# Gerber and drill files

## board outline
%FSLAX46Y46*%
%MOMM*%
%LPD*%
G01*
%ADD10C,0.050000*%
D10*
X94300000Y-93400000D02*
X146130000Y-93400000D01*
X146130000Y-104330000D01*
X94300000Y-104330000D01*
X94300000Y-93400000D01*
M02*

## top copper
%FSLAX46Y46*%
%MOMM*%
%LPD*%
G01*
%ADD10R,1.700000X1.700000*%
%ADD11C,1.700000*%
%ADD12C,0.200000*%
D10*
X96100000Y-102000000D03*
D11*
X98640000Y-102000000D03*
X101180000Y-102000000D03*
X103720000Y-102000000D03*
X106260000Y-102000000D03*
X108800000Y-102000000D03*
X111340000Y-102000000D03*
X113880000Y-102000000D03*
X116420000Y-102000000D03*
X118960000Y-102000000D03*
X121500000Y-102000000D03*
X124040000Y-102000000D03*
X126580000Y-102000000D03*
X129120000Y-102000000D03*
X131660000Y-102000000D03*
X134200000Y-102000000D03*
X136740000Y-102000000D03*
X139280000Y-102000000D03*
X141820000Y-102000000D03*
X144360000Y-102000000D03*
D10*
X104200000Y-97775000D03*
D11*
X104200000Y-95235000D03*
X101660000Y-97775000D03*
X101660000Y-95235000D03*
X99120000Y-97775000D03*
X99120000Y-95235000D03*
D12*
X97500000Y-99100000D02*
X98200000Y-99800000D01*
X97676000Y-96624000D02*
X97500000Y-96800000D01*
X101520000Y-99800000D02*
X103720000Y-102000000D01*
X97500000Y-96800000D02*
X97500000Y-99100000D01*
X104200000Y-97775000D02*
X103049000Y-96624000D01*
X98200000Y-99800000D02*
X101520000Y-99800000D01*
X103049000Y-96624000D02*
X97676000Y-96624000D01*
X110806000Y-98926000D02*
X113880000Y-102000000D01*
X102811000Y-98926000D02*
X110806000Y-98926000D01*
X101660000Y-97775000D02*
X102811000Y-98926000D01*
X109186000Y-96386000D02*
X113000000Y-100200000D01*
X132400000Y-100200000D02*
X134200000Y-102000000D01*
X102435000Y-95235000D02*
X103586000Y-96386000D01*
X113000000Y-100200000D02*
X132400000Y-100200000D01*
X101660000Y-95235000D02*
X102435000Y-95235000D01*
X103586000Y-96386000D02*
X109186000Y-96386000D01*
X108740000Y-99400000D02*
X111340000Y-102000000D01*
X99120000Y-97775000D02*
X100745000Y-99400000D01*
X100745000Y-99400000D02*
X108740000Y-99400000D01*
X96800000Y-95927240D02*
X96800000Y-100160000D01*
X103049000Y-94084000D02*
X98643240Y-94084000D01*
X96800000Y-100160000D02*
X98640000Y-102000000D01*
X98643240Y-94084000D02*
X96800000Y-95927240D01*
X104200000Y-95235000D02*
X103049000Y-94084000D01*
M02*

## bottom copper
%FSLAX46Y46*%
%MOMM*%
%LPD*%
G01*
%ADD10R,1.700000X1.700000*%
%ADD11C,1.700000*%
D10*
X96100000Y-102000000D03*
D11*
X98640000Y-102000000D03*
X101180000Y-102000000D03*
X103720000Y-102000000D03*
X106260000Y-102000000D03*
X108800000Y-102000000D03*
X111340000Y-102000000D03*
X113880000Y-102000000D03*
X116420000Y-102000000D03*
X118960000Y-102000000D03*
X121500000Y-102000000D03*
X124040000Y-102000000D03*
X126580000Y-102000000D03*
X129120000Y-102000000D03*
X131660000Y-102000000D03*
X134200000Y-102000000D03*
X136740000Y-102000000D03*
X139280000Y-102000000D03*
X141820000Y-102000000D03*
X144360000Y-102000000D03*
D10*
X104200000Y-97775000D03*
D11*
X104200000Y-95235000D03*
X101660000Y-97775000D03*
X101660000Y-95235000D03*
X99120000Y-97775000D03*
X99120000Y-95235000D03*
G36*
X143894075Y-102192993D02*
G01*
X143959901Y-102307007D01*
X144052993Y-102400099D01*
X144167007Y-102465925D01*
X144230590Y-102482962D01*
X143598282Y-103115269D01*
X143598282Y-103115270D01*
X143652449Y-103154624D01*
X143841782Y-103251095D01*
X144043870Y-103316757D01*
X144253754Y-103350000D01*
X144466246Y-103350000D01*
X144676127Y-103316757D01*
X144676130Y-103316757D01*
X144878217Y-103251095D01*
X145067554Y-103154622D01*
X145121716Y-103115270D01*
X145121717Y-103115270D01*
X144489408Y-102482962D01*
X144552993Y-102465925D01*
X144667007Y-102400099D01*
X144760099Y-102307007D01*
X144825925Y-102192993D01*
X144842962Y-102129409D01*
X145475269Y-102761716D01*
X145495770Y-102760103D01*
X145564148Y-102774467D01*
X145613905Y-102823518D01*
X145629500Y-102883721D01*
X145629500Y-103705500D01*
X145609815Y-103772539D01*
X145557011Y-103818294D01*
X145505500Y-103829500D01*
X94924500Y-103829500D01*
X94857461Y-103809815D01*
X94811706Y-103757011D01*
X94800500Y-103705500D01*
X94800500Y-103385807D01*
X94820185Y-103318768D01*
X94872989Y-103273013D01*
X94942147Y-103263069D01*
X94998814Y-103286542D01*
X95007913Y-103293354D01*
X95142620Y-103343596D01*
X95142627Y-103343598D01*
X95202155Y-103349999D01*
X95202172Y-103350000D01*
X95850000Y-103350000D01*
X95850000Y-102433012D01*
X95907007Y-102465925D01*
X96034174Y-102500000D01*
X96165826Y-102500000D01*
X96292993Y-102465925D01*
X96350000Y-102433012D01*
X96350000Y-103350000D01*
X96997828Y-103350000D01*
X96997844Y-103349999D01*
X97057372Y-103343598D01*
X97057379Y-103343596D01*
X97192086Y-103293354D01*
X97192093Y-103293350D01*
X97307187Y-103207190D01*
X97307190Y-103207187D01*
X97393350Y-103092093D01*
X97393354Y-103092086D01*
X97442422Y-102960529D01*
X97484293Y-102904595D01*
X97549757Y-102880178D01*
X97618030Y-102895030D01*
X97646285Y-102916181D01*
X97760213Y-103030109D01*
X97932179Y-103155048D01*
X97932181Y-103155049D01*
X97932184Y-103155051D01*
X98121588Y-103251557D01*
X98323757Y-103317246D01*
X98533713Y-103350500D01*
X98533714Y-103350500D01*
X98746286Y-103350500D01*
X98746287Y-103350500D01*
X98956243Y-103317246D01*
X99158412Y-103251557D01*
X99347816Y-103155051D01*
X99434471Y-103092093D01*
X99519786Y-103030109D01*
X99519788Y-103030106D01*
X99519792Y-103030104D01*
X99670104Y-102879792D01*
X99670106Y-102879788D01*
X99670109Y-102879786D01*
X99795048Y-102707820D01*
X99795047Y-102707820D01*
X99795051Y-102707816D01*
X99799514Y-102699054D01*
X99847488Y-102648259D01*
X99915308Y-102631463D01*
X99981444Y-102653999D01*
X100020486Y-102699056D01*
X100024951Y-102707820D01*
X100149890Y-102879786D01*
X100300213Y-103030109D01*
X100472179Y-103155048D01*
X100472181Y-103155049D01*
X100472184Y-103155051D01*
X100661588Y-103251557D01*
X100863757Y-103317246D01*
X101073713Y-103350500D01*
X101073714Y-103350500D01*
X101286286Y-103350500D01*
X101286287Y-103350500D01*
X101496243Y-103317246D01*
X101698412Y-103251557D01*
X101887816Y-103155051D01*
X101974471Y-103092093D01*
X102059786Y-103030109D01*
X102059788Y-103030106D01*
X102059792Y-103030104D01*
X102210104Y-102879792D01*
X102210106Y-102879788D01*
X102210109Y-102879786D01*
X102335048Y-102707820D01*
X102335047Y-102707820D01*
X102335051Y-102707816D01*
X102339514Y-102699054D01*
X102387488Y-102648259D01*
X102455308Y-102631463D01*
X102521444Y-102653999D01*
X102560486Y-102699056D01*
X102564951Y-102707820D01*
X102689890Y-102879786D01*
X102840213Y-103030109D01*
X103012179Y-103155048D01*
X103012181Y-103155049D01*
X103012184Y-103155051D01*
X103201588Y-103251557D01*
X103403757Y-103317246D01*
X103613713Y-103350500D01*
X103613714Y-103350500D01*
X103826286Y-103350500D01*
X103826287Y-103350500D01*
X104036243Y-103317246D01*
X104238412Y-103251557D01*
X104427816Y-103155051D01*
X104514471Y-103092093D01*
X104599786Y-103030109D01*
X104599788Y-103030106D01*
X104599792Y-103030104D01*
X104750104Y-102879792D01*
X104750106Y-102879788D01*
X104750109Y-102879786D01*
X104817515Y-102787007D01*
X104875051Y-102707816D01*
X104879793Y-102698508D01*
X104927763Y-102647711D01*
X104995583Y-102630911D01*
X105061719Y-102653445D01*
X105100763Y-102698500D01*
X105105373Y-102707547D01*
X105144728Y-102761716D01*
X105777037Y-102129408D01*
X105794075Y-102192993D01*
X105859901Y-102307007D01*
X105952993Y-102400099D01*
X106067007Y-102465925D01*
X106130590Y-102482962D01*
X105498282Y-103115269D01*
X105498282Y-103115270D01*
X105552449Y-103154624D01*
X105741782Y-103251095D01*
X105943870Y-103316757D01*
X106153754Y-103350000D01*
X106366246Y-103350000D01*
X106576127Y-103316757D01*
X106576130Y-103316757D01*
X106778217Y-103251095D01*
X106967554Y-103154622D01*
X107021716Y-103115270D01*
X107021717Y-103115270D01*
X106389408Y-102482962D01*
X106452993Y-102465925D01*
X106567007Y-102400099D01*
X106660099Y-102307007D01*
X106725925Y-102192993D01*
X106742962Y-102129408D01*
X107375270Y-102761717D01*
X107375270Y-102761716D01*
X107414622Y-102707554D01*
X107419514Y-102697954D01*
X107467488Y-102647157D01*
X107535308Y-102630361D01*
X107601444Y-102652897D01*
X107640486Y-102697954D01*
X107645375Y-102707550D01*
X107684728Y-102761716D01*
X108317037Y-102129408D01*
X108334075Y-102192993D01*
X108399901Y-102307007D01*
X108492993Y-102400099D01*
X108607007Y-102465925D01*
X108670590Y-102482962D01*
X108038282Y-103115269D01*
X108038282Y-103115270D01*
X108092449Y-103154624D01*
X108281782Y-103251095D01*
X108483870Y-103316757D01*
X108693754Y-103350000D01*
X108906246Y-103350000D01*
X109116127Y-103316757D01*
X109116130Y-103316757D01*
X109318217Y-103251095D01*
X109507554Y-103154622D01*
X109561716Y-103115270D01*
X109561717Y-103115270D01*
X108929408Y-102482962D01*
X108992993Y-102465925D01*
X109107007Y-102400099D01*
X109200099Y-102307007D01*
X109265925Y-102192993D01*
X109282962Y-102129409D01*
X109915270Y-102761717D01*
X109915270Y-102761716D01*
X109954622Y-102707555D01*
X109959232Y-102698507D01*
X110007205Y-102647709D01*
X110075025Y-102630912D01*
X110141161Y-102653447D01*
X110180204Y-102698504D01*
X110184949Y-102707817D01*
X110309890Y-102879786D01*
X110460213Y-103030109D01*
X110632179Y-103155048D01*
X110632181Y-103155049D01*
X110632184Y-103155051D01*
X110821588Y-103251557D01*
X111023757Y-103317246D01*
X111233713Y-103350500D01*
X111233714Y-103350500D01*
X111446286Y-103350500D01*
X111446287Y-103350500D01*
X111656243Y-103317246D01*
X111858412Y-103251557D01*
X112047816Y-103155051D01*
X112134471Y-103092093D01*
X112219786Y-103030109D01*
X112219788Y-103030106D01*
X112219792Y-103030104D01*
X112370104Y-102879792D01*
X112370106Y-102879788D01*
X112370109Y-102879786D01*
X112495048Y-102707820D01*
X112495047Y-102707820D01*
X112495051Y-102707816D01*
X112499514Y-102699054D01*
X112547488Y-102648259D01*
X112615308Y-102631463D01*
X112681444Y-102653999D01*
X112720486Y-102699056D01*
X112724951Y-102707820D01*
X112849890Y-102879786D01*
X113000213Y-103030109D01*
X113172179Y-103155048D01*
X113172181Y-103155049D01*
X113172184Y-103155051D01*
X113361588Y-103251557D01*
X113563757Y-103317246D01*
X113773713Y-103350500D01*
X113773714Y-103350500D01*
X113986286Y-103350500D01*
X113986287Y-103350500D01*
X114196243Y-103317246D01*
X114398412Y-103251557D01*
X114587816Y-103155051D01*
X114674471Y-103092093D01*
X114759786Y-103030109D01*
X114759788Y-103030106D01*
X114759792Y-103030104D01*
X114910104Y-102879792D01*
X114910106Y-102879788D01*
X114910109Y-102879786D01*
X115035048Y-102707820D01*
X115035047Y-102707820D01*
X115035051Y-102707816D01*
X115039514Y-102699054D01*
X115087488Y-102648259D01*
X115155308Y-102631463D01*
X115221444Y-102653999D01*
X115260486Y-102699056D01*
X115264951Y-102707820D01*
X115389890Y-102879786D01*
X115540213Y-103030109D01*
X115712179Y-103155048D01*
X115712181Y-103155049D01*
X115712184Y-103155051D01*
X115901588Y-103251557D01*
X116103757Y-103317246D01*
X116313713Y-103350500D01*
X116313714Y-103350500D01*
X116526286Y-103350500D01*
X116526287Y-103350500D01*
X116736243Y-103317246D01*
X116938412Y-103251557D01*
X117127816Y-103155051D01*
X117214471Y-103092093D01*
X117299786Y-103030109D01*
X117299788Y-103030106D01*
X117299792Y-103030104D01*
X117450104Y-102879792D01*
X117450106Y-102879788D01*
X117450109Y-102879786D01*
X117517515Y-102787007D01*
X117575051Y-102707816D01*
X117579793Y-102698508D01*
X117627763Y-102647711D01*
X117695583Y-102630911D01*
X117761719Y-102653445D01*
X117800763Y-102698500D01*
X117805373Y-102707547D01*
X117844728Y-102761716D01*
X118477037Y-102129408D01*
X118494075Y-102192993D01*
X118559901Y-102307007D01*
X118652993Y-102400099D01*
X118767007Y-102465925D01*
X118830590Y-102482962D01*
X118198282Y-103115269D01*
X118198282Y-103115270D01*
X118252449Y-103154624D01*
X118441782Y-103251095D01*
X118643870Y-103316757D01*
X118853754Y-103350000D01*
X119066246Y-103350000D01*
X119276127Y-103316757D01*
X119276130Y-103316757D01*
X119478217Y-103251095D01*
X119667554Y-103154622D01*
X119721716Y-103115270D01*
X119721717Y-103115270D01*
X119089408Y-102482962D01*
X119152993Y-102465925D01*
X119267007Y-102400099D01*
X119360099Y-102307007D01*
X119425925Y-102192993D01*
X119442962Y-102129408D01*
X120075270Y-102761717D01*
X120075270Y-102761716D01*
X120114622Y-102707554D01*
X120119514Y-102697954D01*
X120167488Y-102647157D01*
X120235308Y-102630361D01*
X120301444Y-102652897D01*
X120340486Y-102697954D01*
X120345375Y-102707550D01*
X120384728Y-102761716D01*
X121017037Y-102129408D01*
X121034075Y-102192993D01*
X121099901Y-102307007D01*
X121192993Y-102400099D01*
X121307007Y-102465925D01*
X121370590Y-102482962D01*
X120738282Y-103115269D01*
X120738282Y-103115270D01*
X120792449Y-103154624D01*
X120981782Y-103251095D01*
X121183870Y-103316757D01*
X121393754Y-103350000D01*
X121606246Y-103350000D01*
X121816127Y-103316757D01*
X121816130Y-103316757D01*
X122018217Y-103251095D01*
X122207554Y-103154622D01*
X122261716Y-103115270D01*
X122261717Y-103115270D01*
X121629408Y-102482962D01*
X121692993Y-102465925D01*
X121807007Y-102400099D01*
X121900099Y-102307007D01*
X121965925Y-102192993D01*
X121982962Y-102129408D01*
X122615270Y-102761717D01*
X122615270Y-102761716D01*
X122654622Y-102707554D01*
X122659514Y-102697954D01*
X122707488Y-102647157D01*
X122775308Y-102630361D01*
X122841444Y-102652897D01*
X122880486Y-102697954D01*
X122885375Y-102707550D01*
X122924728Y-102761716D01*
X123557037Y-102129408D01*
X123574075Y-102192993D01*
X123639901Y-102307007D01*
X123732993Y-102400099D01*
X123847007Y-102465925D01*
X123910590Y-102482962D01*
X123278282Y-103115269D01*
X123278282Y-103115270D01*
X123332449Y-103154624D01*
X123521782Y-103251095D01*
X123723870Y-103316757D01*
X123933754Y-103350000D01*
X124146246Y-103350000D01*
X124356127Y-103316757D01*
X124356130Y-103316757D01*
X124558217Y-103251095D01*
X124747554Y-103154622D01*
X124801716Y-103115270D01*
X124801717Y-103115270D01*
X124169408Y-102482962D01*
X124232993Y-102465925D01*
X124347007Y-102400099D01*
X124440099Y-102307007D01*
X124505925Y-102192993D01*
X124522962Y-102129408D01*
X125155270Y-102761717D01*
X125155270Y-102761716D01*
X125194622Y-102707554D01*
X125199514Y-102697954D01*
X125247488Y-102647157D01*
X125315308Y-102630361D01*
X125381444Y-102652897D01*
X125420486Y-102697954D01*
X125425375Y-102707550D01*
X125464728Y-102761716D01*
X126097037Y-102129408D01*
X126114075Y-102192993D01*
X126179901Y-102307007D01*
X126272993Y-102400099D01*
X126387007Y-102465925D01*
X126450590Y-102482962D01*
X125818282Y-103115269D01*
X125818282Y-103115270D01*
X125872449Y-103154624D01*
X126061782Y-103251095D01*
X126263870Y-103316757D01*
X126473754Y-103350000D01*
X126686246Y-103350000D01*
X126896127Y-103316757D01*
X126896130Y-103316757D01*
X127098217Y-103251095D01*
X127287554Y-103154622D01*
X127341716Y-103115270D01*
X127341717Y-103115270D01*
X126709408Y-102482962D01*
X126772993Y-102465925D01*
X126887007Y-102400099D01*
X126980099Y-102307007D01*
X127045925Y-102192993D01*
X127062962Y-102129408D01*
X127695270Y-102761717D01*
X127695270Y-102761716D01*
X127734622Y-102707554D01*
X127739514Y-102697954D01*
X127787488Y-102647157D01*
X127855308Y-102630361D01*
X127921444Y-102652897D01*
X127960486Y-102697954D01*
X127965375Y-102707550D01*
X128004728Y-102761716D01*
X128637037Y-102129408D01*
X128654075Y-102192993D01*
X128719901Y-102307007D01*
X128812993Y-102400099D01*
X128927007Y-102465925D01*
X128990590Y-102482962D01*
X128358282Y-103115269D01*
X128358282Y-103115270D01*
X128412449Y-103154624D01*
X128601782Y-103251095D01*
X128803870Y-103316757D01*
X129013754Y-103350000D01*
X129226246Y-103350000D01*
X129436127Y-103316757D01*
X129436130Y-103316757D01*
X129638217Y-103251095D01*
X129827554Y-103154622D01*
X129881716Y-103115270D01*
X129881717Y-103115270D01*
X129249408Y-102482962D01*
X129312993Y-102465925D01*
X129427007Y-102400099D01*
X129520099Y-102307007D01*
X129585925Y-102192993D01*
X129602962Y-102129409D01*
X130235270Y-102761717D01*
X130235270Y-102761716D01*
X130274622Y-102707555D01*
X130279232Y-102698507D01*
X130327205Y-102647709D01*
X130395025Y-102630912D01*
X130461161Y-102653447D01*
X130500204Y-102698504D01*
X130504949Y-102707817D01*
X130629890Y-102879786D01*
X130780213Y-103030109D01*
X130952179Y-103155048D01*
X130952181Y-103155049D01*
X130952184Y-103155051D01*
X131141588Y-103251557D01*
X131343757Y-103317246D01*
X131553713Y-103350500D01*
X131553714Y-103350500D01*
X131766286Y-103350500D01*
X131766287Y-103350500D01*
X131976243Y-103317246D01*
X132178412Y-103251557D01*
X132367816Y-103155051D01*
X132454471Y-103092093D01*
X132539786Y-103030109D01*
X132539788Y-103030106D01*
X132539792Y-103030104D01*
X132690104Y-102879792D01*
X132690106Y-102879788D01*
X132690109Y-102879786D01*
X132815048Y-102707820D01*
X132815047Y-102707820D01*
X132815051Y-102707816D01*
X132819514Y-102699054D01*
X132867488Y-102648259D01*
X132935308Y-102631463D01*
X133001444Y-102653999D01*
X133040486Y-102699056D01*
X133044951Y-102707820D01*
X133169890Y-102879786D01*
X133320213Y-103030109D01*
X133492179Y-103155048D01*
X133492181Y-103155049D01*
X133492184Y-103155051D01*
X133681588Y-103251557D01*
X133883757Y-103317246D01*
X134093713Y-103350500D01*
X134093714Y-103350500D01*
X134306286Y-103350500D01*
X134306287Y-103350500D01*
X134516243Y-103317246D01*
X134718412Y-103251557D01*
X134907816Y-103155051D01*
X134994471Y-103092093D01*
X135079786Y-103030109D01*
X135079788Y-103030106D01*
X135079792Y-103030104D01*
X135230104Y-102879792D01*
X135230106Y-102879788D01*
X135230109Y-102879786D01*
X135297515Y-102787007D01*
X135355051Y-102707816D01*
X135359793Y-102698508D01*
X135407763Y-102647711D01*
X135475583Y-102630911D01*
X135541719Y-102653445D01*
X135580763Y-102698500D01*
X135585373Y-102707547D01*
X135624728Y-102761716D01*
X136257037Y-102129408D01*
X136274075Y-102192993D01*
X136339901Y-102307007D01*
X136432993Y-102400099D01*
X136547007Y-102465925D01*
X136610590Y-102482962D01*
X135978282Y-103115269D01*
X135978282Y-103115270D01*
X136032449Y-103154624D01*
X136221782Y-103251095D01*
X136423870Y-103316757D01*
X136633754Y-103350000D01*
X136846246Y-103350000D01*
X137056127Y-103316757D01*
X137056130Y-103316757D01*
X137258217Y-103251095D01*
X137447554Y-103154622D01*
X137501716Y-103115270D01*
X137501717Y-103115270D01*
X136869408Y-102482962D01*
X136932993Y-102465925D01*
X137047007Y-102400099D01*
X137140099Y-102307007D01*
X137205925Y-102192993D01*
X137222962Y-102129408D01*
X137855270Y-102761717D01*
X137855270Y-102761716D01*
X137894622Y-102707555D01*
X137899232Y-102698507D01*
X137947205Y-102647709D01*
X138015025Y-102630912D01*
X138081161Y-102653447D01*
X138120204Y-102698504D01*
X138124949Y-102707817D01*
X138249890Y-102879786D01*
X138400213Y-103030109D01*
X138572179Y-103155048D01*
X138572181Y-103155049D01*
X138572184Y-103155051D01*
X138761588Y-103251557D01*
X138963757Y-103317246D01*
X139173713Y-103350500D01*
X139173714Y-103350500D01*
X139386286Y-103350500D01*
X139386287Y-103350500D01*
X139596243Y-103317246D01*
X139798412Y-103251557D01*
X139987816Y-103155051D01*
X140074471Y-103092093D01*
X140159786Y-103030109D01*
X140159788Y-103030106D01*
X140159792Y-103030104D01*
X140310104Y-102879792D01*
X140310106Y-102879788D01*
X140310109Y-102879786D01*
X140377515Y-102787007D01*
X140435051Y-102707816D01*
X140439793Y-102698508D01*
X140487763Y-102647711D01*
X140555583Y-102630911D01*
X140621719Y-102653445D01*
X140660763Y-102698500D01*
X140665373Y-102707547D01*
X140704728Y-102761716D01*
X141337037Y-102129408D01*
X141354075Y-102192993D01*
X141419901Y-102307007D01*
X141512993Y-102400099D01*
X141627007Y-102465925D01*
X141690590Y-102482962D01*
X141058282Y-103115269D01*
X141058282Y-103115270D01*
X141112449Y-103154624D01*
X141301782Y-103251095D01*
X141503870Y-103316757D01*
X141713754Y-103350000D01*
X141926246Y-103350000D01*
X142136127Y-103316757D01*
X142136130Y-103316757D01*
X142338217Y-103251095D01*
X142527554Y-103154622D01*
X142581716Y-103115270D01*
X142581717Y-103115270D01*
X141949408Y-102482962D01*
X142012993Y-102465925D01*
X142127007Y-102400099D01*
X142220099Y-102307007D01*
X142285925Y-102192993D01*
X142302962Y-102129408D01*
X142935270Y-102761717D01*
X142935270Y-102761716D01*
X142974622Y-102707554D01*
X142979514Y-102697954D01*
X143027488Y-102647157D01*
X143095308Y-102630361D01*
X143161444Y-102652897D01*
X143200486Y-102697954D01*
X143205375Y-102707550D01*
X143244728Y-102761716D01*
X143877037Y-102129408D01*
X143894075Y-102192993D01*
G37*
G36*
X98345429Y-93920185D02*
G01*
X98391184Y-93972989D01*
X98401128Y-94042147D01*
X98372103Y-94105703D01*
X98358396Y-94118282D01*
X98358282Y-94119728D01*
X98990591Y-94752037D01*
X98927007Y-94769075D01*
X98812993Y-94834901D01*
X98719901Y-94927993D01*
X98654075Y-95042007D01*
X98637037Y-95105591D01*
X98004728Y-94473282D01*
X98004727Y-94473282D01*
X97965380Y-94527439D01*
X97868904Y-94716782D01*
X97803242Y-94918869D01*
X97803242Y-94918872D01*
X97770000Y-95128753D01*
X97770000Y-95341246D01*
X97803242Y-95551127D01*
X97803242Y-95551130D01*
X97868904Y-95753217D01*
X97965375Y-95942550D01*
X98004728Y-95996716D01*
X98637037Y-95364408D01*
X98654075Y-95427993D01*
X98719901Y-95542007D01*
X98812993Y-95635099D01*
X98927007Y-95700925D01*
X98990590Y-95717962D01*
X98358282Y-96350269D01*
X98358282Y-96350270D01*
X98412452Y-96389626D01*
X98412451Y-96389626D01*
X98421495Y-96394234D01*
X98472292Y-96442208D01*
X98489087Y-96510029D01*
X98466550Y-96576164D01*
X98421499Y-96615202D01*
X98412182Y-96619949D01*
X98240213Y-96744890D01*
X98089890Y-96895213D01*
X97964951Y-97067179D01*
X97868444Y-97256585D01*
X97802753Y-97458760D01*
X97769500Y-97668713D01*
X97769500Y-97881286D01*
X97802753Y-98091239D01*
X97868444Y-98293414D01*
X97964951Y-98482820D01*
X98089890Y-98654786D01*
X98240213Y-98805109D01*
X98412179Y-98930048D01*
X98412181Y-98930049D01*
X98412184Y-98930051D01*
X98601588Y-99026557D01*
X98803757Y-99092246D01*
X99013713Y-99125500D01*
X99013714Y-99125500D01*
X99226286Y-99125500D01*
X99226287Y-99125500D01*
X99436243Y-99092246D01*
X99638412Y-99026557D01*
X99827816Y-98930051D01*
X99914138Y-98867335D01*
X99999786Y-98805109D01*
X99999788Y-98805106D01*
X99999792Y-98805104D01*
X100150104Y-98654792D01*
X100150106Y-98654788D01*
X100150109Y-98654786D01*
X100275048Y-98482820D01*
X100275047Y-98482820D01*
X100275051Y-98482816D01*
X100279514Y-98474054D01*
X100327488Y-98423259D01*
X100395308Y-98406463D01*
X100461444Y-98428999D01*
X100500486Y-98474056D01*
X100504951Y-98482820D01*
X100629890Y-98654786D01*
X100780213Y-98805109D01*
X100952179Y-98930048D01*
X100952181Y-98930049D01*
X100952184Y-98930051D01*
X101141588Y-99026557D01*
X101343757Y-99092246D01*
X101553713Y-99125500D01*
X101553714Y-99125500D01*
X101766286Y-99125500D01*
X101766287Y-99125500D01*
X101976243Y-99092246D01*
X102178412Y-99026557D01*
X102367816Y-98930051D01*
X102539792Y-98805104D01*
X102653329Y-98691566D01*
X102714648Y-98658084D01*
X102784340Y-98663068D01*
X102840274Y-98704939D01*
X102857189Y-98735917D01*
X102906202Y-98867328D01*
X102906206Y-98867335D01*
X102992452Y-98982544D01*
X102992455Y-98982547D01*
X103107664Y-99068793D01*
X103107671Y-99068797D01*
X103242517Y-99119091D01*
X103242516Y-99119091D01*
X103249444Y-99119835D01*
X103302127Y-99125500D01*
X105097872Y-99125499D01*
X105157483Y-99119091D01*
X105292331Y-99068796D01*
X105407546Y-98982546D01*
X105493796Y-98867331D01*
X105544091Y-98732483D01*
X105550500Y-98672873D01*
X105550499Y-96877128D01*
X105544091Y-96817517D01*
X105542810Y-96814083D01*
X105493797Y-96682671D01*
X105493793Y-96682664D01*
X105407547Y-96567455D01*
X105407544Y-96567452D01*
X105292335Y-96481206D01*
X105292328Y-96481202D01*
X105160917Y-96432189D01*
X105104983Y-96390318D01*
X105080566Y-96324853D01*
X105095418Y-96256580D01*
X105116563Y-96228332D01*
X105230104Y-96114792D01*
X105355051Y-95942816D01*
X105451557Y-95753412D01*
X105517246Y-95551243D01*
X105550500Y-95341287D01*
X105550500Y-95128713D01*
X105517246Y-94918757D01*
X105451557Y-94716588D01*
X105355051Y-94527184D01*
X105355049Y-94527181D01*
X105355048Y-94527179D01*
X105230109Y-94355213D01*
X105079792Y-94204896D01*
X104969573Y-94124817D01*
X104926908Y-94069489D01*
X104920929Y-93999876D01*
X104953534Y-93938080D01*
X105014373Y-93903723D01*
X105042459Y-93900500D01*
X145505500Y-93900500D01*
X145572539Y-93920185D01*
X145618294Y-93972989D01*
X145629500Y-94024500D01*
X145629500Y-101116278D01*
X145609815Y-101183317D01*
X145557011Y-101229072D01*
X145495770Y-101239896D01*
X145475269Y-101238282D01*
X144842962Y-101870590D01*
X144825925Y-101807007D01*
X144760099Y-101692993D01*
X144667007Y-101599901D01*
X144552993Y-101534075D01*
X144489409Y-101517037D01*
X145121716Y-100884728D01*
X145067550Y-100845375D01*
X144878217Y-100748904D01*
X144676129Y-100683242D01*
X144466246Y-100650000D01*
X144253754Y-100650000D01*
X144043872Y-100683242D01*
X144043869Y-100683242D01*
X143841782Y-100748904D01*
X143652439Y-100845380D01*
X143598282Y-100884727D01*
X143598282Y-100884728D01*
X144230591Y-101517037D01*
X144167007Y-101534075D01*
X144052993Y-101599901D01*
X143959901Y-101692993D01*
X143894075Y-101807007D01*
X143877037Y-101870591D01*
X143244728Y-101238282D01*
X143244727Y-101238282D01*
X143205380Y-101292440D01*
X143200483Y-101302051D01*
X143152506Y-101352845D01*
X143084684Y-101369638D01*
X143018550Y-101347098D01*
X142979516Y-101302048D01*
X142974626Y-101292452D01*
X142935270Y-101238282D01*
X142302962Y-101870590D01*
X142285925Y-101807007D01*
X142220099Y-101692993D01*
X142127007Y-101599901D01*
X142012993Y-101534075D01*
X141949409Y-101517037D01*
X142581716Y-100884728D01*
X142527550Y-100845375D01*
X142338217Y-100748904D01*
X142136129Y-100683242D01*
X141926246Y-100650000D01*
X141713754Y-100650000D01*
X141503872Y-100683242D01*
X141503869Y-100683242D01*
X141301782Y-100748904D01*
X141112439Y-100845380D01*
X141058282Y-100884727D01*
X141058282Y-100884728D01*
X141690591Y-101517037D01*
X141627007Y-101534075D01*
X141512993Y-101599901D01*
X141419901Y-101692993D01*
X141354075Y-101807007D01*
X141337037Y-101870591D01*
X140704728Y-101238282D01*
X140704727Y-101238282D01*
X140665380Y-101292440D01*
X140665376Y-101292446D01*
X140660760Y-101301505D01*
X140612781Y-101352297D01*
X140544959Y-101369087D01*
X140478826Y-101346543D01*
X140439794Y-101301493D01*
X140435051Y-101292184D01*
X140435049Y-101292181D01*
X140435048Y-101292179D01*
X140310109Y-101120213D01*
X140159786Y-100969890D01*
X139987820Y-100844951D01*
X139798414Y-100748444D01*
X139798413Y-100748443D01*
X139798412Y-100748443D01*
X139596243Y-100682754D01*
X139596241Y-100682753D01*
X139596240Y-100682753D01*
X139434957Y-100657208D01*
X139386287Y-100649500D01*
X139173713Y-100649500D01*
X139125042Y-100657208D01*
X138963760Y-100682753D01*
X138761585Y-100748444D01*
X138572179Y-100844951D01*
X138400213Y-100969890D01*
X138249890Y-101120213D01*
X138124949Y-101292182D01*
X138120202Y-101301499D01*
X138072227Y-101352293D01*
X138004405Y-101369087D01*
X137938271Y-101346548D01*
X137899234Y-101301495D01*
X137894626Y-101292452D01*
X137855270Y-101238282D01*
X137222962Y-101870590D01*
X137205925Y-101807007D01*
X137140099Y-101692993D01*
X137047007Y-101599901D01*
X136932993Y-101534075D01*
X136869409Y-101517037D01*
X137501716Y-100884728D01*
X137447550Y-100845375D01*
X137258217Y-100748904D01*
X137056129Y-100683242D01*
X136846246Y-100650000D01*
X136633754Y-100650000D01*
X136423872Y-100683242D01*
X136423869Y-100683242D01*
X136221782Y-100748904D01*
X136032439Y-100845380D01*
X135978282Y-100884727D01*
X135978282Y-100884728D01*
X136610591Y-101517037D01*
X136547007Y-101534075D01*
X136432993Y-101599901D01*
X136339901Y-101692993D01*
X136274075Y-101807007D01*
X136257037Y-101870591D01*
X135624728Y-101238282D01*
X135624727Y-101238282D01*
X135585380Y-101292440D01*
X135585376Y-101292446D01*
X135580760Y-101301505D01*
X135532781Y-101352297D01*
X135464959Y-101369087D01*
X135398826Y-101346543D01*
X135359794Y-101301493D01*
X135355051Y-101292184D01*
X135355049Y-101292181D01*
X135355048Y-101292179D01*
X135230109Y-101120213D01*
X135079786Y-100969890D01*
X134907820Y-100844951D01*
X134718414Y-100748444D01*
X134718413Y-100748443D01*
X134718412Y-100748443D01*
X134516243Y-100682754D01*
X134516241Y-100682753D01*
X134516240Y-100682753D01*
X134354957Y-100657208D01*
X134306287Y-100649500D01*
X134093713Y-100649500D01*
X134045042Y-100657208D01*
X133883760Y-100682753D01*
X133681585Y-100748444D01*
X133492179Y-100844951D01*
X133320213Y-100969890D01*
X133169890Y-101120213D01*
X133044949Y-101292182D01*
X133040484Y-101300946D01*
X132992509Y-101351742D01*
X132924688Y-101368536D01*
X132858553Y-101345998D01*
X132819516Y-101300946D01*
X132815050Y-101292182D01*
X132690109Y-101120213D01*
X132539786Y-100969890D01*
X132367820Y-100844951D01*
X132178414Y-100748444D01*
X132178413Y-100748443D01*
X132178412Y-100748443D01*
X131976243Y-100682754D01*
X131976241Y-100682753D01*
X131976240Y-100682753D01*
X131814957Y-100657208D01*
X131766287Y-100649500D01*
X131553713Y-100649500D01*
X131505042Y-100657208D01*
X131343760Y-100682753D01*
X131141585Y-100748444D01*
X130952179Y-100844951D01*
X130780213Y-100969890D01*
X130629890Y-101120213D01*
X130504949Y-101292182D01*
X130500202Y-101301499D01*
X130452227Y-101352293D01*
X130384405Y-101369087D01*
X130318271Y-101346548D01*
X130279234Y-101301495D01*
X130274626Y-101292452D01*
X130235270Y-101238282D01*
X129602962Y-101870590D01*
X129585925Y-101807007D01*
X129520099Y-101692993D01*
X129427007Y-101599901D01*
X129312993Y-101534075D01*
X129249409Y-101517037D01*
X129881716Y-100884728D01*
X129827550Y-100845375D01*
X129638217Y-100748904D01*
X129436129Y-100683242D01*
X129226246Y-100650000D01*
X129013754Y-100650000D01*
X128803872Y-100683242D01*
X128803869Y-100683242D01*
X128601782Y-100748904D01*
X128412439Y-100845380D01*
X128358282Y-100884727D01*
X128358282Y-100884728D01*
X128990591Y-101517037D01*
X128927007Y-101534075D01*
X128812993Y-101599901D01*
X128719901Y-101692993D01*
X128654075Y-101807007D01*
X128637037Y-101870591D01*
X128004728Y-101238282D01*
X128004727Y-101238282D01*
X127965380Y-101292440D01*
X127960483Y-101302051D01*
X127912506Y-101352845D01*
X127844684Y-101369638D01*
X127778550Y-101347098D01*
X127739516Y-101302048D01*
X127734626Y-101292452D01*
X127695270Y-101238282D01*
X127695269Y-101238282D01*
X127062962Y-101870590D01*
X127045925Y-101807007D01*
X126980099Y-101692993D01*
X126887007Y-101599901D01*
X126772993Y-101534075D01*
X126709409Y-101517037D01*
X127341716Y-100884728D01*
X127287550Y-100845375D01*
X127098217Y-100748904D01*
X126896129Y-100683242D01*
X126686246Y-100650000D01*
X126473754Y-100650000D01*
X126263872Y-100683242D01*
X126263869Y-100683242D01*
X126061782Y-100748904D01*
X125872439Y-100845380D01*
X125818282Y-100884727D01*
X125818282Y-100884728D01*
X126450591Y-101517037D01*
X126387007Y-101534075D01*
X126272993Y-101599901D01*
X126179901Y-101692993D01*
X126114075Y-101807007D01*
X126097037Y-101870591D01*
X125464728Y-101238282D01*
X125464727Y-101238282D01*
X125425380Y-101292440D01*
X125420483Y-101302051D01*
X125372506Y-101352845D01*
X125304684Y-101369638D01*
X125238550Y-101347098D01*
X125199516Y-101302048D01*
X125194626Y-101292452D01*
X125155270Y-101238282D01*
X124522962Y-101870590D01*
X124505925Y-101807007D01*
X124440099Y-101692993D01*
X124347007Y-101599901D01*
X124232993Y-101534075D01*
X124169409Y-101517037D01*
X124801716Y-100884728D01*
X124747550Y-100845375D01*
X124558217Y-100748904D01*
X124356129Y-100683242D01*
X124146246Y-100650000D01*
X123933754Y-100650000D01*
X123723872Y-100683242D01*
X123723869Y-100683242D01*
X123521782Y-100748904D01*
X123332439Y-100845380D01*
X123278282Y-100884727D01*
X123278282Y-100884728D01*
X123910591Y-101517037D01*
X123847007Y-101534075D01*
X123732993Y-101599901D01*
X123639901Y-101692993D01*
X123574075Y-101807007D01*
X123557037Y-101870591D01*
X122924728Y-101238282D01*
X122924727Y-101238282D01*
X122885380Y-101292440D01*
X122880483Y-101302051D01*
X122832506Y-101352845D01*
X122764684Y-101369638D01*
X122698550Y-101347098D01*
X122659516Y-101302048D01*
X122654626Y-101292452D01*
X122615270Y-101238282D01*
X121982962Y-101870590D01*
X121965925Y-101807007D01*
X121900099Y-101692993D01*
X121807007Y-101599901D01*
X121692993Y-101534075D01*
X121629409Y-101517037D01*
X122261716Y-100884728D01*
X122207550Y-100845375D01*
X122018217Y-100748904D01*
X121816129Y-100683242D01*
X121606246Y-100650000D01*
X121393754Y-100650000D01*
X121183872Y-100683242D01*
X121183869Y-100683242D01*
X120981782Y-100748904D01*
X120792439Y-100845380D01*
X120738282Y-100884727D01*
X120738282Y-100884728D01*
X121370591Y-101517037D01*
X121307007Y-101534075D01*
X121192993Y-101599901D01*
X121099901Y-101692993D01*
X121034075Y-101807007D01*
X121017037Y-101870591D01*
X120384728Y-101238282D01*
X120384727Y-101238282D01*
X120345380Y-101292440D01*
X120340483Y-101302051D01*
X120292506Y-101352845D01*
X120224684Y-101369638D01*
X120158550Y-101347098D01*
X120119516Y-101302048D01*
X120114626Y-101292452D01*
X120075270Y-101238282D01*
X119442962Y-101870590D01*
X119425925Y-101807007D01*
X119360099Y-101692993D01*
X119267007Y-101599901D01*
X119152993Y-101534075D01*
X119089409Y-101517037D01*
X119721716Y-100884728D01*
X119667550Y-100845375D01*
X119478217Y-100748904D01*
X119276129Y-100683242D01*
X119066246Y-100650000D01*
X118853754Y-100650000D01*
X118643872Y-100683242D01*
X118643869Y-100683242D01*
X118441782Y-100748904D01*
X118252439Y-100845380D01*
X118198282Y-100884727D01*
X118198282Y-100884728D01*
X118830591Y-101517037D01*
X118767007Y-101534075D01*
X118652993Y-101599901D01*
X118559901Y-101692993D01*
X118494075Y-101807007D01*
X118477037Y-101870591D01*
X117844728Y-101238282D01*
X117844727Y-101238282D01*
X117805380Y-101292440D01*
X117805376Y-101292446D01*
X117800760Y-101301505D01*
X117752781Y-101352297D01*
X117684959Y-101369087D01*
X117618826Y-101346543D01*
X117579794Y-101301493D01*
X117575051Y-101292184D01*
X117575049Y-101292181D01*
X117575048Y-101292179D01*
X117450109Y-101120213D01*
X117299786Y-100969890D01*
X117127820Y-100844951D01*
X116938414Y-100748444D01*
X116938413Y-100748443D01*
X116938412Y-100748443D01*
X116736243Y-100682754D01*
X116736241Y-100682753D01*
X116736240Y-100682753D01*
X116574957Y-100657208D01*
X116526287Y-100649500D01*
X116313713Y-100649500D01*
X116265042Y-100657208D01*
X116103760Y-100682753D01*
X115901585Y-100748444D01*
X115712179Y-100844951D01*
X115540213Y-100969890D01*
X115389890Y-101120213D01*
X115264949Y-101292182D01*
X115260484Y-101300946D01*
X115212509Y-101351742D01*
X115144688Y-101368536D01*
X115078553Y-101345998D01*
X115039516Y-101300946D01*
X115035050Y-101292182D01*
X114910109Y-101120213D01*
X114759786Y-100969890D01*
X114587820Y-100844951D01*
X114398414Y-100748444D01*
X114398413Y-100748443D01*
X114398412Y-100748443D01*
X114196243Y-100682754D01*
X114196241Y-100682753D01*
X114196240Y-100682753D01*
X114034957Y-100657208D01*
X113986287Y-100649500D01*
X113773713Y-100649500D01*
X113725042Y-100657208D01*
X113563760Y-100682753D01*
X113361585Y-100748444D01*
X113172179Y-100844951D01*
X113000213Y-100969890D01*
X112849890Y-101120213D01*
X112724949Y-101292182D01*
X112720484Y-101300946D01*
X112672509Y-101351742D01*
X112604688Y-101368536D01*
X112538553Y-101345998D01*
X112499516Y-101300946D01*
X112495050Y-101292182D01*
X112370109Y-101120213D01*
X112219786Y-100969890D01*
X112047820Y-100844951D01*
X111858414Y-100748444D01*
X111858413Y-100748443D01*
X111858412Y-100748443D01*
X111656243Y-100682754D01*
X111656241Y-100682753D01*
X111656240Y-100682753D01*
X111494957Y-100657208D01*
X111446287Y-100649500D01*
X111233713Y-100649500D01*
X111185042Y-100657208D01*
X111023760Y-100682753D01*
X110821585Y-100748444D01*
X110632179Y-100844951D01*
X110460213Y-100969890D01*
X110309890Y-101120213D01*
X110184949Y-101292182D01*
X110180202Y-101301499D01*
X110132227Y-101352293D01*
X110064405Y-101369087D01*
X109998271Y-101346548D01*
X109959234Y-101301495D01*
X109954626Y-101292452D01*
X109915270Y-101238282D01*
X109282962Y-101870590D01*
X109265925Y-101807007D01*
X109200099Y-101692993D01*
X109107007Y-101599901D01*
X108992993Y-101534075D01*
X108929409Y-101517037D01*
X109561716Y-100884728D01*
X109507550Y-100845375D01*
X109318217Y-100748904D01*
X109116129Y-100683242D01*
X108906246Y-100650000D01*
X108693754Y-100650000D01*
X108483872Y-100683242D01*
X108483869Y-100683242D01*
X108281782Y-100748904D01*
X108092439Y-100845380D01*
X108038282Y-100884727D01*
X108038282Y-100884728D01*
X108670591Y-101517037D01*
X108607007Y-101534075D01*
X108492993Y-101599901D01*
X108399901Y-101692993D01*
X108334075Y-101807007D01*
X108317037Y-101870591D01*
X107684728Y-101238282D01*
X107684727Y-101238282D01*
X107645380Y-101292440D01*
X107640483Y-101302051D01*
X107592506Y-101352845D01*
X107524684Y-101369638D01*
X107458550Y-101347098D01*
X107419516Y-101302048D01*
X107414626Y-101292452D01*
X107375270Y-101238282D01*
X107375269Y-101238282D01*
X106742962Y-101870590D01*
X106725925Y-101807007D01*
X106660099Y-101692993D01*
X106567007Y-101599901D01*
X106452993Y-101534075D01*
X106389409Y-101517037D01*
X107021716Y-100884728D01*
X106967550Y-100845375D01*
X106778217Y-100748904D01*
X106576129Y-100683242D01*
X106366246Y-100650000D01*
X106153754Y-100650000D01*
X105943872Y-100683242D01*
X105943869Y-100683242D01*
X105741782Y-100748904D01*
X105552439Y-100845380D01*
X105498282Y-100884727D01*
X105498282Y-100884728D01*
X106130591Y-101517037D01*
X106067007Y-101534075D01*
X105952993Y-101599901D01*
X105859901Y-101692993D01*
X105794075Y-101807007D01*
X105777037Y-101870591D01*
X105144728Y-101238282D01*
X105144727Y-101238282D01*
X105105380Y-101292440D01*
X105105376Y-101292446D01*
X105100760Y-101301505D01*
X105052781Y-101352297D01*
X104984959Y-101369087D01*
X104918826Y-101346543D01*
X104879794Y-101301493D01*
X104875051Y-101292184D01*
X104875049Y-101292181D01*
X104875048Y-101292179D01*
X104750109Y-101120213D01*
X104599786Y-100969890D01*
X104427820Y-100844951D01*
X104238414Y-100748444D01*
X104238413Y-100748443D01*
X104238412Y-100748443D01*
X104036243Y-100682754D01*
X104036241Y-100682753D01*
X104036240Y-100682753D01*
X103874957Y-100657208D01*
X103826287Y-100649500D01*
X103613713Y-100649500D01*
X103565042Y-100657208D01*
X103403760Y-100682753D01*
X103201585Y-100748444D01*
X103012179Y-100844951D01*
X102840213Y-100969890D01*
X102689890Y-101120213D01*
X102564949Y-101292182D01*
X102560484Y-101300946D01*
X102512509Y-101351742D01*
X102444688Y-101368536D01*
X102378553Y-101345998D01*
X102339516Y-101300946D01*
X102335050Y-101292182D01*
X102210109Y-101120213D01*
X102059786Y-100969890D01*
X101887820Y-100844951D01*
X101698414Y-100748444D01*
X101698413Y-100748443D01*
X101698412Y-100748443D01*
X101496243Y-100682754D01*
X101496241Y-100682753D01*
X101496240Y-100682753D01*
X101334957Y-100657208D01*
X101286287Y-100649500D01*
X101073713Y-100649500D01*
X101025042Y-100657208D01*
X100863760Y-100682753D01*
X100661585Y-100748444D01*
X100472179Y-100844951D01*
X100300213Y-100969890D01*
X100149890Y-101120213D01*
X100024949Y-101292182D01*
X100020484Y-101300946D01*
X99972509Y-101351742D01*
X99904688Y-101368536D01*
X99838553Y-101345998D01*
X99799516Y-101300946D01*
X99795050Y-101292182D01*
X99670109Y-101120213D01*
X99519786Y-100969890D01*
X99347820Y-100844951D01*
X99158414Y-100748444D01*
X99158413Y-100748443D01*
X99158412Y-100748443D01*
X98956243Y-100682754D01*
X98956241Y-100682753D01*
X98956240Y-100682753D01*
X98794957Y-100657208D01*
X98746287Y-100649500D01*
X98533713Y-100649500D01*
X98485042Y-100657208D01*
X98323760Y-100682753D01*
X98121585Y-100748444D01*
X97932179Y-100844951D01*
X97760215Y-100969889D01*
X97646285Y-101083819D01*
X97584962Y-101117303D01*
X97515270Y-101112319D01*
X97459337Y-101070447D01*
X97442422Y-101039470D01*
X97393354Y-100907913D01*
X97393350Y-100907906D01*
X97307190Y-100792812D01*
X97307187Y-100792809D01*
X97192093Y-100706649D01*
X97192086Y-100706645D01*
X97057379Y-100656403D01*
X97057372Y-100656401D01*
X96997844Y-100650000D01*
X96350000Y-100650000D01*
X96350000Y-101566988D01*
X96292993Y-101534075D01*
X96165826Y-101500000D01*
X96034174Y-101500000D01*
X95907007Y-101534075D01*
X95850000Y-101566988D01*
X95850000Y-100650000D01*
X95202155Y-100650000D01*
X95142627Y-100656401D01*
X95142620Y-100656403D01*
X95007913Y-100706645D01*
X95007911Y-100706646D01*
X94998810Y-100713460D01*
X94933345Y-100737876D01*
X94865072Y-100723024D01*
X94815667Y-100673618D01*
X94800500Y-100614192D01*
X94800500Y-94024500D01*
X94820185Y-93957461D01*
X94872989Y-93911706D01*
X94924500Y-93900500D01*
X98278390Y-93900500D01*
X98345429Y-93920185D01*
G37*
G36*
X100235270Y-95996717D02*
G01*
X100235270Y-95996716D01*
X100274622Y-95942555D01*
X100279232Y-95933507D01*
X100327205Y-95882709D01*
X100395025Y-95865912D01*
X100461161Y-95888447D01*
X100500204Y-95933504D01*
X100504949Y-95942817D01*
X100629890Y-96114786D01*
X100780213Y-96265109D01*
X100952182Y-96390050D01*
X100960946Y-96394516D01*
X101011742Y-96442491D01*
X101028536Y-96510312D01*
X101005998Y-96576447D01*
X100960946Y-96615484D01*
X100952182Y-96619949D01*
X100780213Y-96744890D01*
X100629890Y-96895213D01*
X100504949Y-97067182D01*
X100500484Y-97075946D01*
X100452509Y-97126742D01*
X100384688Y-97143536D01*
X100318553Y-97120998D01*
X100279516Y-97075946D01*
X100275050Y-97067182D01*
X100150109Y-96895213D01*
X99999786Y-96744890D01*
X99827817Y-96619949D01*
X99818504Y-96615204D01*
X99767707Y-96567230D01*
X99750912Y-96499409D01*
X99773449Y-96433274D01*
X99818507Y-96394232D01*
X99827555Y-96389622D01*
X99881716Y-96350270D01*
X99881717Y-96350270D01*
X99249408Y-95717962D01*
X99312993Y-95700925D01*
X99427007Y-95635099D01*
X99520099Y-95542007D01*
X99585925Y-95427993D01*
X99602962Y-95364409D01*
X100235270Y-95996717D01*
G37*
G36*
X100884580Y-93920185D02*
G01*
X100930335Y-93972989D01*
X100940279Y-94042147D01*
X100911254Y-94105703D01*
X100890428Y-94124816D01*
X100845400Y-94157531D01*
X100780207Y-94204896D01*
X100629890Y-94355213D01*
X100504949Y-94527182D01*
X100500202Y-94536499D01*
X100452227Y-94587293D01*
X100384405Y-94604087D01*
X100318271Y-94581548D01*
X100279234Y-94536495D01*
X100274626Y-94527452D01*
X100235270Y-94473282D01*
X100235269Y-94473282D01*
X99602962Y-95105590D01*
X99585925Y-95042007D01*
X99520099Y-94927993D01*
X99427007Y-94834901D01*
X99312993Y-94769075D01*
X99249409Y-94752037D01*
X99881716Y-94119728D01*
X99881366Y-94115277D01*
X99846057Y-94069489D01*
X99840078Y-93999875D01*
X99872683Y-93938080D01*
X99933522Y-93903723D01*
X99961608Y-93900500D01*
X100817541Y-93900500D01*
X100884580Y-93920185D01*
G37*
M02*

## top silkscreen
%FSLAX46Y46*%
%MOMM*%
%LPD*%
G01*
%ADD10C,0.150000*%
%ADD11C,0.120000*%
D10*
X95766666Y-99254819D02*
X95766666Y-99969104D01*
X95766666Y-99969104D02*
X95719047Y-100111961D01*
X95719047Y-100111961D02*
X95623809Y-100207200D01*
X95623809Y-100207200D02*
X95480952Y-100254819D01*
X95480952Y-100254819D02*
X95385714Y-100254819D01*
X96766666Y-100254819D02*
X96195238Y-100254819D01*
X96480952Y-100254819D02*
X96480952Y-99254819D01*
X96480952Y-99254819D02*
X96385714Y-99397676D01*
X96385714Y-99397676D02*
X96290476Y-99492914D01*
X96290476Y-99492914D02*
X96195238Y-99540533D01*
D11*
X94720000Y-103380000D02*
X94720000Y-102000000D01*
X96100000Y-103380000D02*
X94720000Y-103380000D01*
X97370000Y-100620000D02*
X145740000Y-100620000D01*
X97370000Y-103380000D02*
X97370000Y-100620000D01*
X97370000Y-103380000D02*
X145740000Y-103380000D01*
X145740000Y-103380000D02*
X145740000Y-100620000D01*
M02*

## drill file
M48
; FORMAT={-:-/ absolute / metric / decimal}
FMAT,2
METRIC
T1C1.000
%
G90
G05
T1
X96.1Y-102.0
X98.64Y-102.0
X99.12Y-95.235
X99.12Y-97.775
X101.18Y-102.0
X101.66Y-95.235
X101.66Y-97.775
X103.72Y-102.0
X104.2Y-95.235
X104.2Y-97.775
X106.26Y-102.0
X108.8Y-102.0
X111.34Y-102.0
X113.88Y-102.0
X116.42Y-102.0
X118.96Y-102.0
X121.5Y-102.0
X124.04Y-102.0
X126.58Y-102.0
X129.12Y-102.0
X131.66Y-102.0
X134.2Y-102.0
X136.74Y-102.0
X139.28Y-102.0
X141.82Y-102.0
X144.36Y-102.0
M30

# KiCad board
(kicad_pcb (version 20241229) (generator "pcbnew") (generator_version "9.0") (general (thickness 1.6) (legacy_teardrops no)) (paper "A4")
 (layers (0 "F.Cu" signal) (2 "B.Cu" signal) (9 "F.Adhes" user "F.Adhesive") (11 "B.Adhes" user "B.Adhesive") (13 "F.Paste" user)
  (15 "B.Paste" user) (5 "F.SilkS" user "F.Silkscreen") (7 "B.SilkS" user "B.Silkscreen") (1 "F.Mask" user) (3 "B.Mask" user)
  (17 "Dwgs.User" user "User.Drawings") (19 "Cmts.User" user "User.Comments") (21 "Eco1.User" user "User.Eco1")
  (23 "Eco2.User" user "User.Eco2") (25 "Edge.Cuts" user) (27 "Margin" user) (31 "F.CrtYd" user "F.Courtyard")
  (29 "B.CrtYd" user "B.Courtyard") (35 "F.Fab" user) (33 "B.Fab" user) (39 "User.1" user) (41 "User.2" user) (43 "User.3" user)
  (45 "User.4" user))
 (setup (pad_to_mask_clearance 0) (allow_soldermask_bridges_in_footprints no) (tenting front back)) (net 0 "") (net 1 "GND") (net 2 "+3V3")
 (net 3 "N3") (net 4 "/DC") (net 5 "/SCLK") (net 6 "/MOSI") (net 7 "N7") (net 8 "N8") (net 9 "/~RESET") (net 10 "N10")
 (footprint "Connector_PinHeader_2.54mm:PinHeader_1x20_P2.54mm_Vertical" (layer "F.Cu") (at 96.1 102 90)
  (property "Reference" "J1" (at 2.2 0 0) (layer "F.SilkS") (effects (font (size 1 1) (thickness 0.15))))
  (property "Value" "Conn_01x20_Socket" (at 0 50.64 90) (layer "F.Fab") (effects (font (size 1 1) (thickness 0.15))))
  (fp_line (start -1.38 -1.38) (end 0 -1.38) (stroke (width 0.12) (type solid)) (layer "F.SilkS"))
  (fp_line (start -1.38 0) (end -1.38 -1.38) (stroke (width 0.12) (type solid)) (layer "F.SilkS"))
  (fp_line (start 1.38 1.27) (end 1.38 49.64) (stroke (width 0.12) (type solid)) (layer "F.SilkS"))
  (fp_line (start -1.38 1.27) (end 1.38 1.27) (stroke (width 0.12) (type solid)) (layer "F.SilkS"))
  (fp_line (start -1.38 1.27) (end -1.38 49.64) (stroke (width 0.12) (type solid)) (layer "F.SilkS"))
  (fp_line (start -1.38 49.64) (end 1.38 49.64) (stroke (width 0.12) (type solid)) (layer "F.SilkS"))
  (pad "1" thru_hole rect (at 0 0 90) (size 1.7 1.7) (drill 1) (layers "*.Cu" "*.Mask") (remove_unused_layers no) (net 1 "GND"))
  (pad "2" thru_hole circle (at 0 2.54 90) (size 1.7 1.7) (drill 1) (layers "*.Cu" "*.Mask") (remove_unused_layers no) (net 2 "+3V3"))
  (pad "3" thru_hole circle (at 0 5.08 90) (size 1.7 1.7) (drill 1) (layers "*.Cu" "*.Mask") (remove_unused_layers no) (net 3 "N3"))
  (pad "4" thru_hole circle (at 0 7.62 90) (size 1.7 1.7) (drill 1) (layers "*.Cu" "*.Mask") (remove_unused_layers no) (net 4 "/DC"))
  (pad "5" thru_hole circle (at 0 10.16 90) (size 1.7 1.7) (drill 1) (layers "*.Cu" "*.Mask") (remove_unused_layers no) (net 1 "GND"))
  (pad "6" thru_hole circle (at 0 12.7 90) (size 1.7 1.7) (drill 1) (layers "*.Cu" "*.Mask") (remove_unused_layers no) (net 1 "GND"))
  (pad "7" thru_hole circle (at 0 15.24 90) (size 1.7 1.7) (drill 1) (layers "*.Cu" "*.Mask") (remove_unused_layers no) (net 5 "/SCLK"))
  (pad "8" thru_hole circle (at 0 17.78 90) (size 1.7 1.7) (drill 1) (layers "*.Cu" "*.Mask") (remove_unused_layers no) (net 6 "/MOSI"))
  (pad "9" thru_hole circle (at 0 20.32 90) (size 1.7 1.7) (drill 1) (layers "*.Cu" "*.Mask") (remove_unused_layers no) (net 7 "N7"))
  (pad "10" thru_hole circle (at 0 22.86 90) (size 1.7 1.7) (drill 1) (layers "*.Cu" "*.Mask") (remove_unused_layers no) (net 1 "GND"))
  (pad "11" thru_hole circle (at 0 25.4 90) (size 1.7 1.7) (drill 1) (layers "*.Cu" "*.Mask") (remove_unused_layers no) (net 1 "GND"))
  (pad "12" thru_hole circle (at 0 27.94 90) (size 1.7 1.7) (drill 1) (layers "*.Cu" "*.Mask") (remove_unused_layers no) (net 1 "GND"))
  (pad "13" thru_hole circle (at 0 30.48 90) (size 1.7 1.7) (drill 1) (layers "*.Cu" "*.Mask") (remove_unused_layers no) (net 1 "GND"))
  (pad "14" thru_hole circle (at 0 33.02 90) (size 1.7 1.7) (drill 1) (layers "*.Cu" "*.Mask") (remove_unused_layers no) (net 1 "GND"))
  (pad "15" thru_hole circle (at 0 35.56 90) (size 1.7 1.7) (drill 1) (layers "*.Cu" "*.Mask") (remove_unused_layers no) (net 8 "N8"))
  (pad "16" thru_hole circle (at 0 38.1 90) (size 1.7 1.7) (drill 1) (layers "*.Cu" "*.Mask") (remove_unused_layers no) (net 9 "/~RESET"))
  (pad "17" thru_hole circle (at 0 40.64 90) (size 1.7 1.7) (drill 1) (layers "*.Cu" "*.Mask") (remove_unused_layers no) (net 1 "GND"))
  (pad "18" thru_hole circle (at 0 43.18 90) (size 1.7 1.7) (drill 1) (layers "*.Cu" "*.Mask") (remove_unused_layers no) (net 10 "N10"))
  (pad "19" thru_hole circle (at 0 45.72 90) (size 1.7 1.7) (drill 1) (layers "*.Cu" "*.Mask") (remove_unused_layers no) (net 1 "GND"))
  (pad "20" thru_hole circle (at 0 48.26 90) (size 1.7 1.7) (drill 1) (layers "*.Cu" "*.Mask") (remove_unused_layers no) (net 1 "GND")))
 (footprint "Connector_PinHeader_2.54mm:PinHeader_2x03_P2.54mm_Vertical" (layer "B.Cu") (at 104.2 97.775 90)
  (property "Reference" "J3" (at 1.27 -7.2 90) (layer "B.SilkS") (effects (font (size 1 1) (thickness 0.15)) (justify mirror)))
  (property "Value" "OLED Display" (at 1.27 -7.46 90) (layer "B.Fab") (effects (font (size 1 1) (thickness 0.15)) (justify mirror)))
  (pad "1" thru_hole rect (at 0 0 90) (size 1.7 1.7) (drill 1) (layers "*.Cu" "*.Mask") (remove_unused_layers no) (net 4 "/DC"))
  (pad "2" thru_hole circle (at 2.54 0 90) (size 1.7 1.7) (drill 1) (layers "*.Cu" "*.Mask") (remove_unused_layers no) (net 2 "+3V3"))
  (pad "3" thru_hole circle (at 0 -2.54 90) (size 1.7 1.7) (drill 1) (layers "*.Cu" "*.Mask") (remove_unused_layers no) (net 6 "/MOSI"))
  (pad "4" thru_hole circle (at 2.54 -2.54 90) (size 1.7 1.7) (drill 1) (layers "*.Cu" "*.Mask") (remove_unused_layers no) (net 9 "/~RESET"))
  (pad "5" thru_hole circle (at 0 -5.08 90) (size 1.7 1.7) (drill 1) (layers "*.Cu" "*.Mask") (remove_unused_layers no) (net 5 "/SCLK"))
  (pad "6" thru_hole circle (at 2.54 -5.08 90) (size 1.7 1.7) (drill 1) (layers "*.Cu" "*.Mask") (remove_unused_layers no) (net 1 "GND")))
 (gr_rect (start 94.3 93.4) (end 146.13 104.33) (stroke (width 0.05) (type default)) (fill no) (layer "Edge.Cuts"))
 (segment (start 97.5 99.1) (end 98.2 99.8) (width 0.2) (layer "F.Cu") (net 4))
 (segment (start 97.676 96.624) (end 97.5 96.8) (width 0.2) (layer "F.Cu") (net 4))
 (segment (start 101.52 99.8) (end 103.72 102) (width 0.2) (layer "F.Cu") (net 4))
 (segment (start 97.5 96.8) (end 97.5 99.1) (width 0.2) (layer "F.Cu") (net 4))
 (segment (start 104.2 97.775) (end 103.049 96.624) (width 0.2) (layer "F.Cu") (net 4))
 (segment (start 98.2 99.8) (end 101.52 99.8) (width 0.2) (layer "F.Cu") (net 4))
 (segment (start 103.049 96.624) (end 97.676 96.624) (width 0.2) (layer "F.Cu") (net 4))
 (segment (start 110.806 98.926) (end 113.88 102) (width 0.2) (layer "F.Cu") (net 6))
 (segment (start 102.811 98.926) (end 110.806 98.926) (width 0.2) (layer "F.Cu") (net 6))
 (segment (start 101.66 97.775) (end 102.811 98.926) (width 0.2) (layer "F.Cu") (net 6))
 (segment (start 109.186 96.386) (end 113 100.2) (width 0.2) (layer "F.Cu") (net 9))
 (segment (start 132.4 100.2) (end 134.2 102) (width 0.2) (layer "F.Cu") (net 9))
 (segment (start 102.435 95.235) (end 103.586 96.386) (width 0.2) (layer "F.Cu") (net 9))
 (segment (start 113 100.2) (end 132.4 100.2) (width 0.2) (layer "F.Cu") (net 9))
 (segment (start 101.66 95.235) (end 102.435 95.235) (width 0.2) (layer "F.Cu") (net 9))
 (segment (start 103.586 96.386) (end 109.186 96.386) (width 0.2) (layer "F.Cu") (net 9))
 (segment (start 108.74 99.4) (end 111.34 102) (width 0.2) (layer "F.Cu") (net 5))
 (segment (start 99.12 97.775) (end 100.745 99.4) (width 0.2) (layer "F.Cu") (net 5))
 (segment (start 100.745 99.4) (end 108.74 99.4) (width 0.2) (layer "F.Cu") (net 5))
 (segment (start 96.8 95.92724) (end 96.8 100.16) (width 0.2) (layer "F.Cu") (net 2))
 (segment (start 103.049 94.084) (end 98.64324 94.084) (width 0.2) (layer "F.Cu") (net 2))
 (segment (start 96.8 100.16) (end 98.64 102) (width 0.2) (layer "F.Cu") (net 2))
 (segment (start 98.64324 94.084) (end 96.8 95.92724) (width 0.2) (layer "F.Cu") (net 2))
 (segment (start 104.2 95.235) (end 103.049 94.084) (width 0.2) (layer "F.Cu") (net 2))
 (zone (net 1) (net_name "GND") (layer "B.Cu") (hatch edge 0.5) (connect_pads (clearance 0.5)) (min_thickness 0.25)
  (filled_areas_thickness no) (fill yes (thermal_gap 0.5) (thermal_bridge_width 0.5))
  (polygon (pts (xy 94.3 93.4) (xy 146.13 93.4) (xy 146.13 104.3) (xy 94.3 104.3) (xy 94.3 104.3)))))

